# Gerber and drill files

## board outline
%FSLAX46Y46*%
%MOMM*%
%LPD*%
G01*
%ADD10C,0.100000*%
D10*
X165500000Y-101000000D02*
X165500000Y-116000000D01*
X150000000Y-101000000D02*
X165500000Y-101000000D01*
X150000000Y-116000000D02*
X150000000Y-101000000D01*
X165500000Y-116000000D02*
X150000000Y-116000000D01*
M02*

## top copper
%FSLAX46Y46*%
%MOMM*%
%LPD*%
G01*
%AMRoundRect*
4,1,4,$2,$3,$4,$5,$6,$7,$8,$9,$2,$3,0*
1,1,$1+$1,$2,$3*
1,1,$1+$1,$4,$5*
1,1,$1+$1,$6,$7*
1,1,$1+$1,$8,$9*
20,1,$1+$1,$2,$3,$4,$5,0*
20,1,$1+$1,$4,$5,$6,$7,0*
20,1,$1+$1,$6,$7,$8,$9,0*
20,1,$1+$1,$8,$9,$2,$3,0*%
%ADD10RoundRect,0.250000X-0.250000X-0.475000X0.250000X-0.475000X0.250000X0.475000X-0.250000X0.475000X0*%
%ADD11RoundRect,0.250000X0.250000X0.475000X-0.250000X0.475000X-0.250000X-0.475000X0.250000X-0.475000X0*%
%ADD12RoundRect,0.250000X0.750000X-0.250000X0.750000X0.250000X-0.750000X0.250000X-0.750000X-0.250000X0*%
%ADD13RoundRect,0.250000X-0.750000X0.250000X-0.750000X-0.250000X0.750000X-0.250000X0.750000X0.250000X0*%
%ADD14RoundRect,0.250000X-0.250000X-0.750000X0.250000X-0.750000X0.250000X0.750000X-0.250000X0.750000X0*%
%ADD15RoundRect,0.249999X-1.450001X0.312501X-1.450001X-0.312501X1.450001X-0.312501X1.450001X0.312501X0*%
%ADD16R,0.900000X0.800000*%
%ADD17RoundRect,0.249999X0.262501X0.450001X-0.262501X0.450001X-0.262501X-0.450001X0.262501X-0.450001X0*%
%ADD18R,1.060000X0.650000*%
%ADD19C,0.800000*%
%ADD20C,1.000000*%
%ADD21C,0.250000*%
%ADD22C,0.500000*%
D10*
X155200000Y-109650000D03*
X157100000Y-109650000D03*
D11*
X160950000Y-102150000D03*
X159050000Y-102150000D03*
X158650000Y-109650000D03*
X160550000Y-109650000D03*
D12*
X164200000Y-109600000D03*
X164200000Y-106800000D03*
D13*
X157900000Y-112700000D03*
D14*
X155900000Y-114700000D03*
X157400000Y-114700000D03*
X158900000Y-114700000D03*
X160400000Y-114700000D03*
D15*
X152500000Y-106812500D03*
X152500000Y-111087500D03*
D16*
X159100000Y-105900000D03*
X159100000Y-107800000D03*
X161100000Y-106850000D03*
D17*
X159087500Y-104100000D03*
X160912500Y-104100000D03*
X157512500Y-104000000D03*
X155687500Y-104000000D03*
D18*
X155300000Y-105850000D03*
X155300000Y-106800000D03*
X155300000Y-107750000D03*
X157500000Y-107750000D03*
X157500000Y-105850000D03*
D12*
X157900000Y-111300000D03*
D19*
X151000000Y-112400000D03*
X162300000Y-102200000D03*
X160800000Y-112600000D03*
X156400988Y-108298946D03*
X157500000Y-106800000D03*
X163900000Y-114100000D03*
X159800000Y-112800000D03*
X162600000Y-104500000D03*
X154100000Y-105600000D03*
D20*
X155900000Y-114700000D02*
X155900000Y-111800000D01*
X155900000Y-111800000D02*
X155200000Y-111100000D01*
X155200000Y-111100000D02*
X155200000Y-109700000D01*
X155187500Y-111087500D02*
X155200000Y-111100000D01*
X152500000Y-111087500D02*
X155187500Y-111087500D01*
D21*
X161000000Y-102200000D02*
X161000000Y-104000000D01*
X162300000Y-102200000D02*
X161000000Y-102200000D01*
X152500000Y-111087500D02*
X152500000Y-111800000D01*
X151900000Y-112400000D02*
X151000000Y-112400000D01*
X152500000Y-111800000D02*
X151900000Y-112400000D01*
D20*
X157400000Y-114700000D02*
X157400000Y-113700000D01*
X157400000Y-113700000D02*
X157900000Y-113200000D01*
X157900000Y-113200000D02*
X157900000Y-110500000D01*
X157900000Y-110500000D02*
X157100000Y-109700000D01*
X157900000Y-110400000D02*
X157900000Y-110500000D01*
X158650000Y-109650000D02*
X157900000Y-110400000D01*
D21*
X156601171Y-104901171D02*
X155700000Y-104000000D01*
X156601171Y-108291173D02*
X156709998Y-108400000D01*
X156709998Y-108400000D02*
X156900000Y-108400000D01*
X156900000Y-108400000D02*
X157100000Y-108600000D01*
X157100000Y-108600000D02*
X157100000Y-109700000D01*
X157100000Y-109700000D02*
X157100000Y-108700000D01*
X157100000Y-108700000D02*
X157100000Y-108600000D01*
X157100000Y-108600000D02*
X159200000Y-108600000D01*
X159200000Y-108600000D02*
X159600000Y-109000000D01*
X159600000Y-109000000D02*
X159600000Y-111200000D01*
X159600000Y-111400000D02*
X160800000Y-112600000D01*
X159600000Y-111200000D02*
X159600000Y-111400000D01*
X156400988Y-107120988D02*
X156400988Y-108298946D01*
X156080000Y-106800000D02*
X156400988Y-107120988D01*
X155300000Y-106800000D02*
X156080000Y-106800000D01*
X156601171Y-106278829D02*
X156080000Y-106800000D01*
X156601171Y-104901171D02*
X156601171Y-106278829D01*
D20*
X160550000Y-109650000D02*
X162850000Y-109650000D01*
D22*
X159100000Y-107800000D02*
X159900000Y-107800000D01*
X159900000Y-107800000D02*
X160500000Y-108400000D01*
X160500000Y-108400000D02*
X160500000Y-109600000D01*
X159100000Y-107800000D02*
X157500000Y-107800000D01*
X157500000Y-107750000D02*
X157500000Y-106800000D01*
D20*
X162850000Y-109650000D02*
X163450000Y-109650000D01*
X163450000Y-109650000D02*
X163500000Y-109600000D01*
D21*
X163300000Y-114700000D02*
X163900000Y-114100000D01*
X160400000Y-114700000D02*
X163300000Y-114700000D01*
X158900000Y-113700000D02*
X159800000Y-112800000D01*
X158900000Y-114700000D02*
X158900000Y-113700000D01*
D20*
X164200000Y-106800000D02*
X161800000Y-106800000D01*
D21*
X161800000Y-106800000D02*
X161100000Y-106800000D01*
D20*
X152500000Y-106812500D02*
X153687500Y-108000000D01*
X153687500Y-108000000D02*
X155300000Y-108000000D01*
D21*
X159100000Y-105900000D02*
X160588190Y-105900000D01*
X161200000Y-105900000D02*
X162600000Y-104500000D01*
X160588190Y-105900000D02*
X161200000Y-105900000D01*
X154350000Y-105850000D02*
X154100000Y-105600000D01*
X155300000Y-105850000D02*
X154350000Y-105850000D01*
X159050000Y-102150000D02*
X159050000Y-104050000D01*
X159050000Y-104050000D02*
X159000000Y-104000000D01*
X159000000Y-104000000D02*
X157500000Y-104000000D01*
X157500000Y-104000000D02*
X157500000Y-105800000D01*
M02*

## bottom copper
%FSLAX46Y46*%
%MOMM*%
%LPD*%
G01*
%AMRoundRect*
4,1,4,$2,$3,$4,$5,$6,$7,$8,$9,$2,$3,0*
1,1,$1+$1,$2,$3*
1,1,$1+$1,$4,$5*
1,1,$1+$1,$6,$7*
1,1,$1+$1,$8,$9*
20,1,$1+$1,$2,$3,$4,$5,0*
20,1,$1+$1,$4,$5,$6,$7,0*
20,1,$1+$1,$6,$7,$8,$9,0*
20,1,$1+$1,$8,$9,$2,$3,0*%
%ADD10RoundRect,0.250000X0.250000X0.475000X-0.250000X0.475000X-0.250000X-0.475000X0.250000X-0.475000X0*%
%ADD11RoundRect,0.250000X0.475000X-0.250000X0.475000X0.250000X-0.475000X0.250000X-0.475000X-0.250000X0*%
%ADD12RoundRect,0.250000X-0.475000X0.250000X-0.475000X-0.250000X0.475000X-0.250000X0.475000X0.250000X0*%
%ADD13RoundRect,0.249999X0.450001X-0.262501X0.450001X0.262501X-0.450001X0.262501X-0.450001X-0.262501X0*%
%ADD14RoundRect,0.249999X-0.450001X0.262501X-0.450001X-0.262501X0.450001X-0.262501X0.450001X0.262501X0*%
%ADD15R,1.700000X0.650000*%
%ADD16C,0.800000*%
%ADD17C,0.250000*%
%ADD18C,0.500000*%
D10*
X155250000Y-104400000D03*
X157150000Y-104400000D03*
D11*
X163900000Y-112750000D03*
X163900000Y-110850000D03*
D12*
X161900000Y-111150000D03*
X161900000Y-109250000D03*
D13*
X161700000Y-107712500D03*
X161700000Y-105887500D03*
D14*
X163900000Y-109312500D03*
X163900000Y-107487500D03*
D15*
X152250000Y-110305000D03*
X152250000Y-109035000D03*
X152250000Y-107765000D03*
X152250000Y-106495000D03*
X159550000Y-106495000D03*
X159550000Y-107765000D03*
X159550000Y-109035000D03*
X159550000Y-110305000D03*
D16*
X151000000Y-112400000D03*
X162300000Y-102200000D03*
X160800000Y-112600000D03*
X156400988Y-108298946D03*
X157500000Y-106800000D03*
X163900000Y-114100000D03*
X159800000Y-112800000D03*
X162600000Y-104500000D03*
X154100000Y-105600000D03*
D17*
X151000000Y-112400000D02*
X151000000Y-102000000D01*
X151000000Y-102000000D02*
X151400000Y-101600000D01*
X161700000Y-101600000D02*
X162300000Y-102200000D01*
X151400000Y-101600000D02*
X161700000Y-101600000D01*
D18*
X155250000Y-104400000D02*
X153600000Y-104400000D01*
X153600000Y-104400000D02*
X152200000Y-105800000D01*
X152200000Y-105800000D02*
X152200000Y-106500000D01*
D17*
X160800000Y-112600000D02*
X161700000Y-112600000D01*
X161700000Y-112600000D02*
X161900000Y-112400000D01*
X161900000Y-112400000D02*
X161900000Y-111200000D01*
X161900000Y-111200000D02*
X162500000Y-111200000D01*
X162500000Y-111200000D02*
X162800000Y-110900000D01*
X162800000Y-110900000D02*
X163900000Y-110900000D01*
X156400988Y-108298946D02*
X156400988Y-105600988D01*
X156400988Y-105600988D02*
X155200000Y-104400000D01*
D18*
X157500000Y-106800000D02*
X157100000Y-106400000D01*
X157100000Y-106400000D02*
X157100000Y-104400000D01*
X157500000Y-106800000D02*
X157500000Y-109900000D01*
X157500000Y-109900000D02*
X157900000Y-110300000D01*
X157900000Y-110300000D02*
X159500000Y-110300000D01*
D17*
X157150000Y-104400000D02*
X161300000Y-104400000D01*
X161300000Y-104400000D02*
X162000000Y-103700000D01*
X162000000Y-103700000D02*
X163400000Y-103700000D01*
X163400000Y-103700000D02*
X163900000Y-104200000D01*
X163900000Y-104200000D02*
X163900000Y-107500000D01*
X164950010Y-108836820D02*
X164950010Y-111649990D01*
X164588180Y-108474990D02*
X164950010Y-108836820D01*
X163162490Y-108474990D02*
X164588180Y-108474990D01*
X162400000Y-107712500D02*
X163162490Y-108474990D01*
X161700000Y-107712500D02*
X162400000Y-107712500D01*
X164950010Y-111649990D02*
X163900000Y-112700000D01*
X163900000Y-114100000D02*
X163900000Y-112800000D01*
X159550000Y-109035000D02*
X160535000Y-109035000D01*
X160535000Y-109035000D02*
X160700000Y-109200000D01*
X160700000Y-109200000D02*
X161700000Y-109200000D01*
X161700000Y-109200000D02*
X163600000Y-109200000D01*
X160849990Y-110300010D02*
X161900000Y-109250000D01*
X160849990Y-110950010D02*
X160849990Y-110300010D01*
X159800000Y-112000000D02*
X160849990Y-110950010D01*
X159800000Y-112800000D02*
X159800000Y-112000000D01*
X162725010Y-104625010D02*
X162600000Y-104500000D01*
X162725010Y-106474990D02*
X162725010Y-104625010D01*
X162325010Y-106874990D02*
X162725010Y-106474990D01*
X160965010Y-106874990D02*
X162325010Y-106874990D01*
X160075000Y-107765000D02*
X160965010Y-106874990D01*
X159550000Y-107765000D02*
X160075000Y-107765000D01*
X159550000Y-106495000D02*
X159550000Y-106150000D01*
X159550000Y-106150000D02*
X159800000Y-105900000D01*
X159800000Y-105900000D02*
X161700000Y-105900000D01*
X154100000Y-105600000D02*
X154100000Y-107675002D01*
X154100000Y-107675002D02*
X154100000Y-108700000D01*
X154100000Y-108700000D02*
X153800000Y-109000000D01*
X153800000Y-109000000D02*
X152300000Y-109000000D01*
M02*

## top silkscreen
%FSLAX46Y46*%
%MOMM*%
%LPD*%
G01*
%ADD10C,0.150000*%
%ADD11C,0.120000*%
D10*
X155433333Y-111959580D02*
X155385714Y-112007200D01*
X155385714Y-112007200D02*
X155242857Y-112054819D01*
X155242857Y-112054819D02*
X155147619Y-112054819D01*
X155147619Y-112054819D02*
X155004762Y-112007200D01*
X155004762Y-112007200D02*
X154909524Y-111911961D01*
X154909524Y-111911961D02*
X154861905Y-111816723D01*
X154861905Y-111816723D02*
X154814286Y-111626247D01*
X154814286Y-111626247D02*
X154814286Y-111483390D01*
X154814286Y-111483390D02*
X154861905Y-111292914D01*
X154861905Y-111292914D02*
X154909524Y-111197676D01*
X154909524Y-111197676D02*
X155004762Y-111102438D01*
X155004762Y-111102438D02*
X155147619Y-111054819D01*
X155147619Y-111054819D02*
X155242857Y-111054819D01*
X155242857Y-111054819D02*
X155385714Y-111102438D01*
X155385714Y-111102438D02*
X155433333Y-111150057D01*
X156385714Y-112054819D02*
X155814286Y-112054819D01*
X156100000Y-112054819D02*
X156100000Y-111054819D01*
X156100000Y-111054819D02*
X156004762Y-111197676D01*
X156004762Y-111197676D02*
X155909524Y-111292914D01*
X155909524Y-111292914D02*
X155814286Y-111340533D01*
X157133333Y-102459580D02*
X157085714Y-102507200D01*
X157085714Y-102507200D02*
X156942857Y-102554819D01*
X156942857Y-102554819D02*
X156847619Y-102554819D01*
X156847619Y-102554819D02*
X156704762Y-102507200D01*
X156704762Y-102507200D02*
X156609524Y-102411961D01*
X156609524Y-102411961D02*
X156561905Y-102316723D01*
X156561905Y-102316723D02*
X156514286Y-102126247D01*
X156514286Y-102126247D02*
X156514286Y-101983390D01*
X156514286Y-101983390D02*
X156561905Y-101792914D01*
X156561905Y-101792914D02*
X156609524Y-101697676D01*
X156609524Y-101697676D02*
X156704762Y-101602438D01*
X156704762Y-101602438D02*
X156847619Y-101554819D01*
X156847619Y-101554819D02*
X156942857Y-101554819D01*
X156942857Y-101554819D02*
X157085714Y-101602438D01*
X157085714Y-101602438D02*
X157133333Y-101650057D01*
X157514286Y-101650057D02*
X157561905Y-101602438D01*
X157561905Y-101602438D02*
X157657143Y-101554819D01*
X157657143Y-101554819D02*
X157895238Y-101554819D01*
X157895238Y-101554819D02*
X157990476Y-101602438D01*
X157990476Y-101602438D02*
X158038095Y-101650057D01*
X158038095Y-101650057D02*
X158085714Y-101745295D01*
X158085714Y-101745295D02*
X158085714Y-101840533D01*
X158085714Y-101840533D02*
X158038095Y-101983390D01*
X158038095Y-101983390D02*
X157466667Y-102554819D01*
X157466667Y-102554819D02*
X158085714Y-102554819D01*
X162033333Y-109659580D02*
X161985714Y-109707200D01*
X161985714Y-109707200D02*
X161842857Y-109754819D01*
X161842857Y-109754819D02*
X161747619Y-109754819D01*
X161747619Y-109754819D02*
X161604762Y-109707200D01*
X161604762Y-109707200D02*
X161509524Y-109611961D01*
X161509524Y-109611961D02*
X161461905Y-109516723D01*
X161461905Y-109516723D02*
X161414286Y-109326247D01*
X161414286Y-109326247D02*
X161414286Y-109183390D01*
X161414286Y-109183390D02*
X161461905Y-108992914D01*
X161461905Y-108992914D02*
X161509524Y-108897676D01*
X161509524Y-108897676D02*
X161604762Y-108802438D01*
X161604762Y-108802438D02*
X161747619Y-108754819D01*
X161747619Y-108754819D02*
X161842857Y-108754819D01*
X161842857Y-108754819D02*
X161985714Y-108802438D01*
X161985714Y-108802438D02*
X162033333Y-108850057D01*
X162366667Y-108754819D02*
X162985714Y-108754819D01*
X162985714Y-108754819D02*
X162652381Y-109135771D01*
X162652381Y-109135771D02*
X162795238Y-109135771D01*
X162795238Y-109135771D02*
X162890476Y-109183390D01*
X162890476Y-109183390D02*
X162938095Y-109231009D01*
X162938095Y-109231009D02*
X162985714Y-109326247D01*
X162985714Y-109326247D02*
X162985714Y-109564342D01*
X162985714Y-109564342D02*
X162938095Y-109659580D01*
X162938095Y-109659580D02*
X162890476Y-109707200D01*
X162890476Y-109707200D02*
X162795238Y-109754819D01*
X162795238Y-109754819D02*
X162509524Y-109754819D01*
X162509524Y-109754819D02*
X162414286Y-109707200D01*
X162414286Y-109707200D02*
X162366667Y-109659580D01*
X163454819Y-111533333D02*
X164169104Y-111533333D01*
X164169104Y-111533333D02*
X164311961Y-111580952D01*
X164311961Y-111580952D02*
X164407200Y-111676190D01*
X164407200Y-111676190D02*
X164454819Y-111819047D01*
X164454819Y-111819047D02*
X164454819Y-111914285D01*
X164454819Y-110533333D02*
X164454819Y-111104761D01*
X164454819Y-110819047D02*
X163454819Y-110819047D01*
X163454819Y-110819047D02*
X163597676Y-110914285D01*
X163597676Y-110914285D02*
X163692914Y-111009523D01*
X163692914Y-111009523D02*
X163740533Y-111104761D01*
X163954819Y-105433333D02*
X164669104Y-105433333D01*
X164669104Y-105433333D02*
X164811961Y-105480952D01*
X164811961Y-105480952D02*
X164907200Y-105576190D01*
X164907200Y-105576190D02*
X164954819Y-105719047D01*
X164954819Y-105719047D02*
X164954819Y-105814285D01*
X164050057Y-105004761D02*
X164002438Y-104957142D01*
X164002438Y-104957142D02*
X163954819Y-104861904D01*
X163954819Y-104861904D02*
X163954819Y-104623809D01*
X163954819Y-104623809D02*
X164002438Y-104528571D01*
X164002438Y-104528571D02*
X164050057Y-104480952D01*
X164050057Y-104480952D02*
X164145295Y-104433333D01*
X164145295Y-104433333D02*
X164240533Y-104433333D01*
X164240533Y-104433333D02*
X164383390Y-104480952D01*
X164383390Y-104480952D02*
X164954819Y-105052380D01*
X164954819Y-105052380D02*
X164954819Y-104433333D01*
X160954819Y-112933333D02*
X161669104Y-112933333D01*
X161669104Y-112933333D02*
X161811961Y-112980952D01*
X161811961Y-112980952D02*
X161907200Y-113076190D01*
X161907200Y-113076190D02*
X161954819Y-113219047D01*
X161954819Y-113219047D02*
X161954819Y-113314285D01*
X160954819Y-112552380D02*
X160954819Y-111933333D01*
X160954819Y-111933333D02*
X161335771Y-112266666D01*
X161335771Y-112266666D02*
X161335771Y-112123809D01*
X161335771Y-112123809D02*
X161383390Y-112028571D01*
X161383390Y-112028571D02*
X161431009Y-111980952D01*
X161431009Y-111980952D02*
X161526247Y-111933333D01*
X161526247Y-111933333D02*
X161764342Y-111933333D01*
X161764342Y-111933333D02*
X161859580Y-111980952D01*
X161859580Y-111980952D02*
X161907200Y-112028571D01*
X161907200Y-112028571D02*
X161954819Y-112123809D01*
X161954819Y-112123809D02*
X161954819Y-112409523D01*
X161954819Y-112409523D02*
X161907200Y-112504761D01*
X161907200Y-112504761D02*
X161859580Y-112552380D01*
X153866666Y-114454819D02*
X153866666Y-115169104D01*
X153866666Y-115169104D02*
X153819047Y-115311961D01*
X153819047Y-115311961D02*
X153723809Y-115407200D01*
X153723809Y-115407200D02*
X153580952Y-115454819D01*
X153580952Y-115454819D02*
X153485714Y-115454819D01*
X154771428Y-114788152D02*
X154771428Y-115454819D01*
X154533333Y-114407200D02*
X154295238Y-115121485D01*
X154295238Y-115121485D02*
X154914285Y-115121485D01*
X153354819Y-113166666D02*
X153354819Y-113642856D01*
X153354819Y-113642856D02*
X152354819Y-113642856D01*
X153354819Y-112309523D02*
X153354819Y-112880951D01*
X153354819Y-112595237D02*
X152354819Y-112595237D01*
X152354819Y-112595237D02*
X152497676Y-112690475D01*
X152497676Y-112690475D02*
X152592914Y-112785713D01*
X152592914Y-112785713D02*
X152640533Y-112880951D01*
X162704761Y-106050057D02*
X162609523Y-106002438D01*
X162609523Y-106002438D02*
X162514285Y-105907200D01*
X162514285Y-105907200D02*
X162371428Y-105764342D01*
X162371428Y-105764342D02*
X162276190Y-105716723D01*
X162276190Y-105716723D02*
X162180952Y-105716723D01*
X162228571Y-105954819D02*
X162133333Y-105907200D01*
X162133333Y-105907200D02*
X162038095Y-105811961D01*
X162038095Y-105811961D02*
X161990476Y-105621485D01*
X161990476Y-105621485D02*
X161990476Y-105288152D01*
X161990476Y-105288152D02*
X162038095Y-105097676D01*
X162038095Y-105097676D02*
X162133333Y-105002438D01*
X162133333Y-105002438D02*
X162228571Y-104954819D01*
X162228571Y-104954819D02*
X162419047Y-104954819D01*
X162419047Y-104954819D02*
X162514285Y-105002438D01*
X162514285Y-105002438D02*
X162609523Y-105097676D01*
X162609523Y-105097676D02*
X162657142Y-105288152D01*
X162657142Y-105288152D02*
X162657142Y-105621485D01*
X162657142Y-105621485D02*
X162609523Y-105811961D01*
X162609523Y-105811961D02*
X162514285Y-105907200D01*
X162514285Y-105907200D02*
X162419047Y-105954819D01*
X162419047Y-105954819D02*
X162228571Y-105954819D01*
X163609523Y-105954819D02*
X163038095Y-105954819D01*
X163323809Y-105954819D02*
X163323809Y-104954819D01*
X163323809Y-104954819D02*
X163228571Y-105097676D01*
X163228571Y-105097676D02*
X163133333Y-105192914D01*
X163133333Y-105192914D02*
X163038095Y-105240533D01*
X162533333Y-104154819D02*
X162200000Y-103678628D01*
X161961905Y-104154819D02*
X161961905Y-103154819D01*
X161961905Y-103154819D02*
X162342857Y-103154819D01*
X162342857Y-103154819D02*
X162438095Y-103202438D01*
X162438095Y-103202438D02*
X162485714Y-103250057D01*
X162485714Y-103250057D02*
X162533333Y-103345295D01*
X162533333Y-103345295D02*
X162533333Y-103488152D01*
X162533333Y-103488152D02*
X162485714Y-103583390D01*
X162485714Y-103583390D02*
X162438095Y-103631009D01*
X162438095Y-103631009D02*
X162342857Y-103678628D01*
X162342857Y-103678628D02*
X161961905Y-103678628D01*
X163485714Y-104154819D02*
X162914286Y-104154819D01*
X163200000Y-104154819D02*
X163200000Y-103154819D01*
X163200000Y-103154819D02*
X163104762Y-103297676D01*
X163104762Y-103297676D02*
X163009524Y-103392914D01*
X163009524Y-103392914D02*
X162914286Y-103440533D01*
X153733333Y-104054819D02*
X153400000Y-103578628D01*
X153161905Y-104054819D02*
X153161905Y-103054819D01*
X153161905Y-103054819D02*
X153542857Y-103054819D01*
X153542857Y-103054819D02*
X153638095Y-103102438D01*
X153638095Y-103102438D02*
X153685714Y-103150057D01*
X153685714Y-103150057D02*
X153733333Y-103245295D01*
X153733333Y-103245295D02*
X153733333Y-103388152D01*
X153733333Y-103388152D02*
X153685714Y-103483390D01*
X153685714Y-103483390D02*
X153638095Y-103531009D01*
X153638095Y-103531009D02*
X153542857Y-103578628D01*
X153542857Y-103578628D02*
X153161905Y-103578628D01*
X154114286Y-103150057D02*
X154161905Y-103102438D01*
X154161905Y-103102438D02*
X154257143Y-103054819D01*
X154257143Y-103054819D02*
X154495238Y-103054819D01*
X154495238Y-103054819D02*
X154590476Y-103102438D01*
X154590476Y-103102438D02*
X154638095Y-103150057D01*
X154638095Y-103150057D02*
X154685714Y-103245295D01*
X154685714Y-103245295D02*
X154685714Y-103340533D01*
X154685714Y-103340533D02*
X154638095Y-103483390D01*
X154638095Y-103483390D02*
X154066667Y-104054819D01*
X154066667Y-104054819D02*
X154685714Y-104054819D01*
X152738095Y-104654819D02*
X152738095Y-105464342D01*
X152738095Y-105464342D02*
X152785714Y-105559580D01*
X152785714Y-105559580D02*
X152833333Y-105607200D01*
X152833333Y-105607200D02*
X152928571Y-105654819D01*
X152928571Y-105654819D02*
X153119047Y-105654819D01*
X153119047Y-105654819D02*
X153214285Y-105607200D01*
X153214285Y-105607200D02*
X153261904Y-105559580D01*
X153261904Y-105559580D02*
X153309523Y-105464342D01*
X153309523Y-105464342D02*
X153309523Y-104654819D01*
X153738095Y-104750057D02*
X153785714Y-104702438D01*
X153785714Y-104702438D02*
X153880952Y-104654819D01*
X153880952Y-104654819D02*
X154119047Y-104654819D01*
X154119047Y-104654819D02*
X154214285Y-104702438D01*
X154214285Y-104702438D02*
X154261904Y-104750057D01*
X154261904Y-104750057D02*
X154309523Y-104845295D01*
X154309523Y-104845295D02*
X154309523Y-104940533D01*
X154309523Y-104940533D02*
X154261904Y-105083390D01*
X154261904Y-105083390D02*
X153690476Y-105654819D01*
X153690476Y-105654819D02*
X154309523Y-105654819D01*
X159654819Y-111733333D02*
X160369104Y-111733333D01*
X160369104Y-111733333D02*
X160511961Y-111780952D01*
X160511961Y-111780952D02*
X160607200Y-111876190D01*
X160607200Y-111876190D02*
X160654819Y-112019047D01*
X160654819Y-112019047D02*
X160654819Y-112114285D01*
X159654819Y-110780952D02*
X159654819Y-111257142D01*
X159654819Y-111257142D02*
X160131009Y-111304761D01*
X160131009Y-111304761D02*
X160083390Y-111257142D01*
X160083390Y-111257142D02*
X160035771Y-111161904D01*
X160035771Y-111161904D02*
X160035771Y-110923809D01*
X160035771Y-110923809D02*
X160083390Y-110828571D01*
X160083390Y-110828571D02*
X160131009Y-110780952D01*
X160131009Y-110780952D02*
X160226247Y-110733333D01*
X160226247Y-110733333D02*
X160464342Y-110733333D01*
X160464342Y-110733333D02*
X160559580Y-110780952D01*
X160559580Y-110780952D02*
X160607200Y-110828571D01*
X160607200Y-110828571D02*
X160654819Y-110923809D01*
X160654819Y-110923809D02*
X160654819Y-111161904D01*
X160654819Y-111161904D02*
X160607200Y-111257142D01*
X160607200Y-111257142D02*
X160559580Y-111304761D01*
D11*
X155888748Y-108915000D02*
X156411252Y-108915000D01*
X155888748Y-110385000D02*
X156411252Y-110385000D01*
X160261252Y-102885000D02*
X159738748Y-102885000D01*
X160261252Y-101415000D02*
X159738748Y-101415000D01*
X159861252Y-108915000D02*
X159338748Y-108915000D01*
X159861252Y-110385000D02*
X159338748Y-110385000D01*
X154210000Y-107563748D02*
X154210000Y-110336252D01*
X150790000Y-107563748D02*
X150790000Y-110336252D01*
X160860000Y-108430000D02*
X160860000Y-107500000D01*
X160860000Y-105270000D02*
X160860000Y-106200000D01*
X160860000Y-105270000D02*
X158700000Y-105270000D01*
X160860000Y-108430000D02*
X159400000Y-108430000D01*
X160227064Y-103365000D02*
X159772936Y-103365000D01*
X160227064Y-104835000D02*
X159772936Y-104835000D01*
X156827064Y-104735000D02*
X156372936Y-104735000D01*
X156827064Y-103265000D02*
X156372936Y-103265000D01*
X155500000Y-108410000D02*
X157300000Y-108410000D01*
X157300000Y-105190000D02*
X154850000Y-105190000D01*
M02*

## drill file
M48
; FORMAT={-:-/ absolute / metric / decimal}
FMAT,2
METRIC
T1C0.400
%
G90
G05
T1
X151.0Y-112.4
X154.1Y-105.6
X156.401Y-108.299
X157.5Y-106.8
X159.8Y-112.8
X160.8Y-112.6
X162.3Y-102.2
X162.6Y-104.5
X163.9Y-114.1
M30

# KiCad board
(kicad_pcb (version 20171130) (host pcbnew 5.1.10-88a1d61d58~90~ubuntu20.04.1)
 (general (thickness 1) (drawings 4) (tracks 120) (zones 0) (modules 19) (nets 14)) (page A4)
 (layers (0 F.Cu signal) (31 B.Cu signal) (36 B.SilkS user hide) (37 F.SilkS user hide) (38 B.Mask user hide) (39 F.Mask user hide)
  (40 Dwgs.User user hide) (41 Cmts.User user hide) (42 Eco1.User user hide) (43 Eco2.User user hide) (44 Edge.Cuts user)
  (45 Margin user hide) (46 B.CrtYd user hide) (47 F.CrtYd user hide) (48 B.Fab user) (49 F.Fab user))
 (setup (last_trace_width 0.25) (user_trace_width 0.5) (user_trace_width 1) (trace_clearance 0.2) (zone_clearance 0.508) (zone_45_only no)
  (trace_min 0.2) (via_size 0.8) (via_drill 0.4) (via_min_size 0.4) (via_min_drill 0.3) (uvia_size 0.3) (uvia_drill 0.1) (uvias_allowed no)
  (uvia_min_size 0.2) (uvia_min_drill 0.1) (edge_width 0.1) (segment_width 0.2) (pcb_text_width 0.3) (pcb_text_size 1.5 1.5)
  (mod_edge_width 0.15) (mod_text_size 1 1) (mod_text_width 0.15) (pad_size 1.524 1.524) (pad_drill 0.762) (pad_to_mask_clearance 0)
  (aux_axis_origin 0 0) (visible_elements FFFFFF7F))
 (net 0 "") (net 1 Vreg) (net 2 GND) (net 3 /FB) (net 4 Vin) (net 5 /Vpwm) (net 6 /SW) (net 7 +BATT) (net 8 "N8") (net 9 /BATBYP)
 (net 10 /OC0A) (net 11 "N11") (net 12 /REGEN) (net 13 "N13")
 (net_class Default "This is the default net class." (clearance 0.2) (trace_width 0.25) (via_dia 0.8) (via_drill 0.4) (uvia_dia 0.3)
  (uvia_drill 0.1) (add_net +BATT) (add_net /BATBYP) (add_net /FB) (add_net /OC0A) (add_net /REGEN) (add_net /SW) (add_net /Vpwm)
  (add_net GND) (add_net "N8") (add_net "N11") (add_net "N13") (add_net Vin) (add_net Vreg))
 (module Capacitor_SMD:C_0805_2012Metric (layer F.Cu) (at 156.15 109.65)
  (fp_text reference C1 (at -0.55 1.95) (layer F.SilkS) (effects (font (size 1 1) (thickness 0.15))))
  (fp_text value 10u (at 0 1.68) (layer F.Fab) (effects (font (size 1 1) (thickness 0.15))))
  (fp_line (start -0.261252 -0.735) (end 0.261252 -0.735) (layer F.SilkS) (width 0.12))
  (fp_line (start -0.261252 0.735) (end 0.261252 0.735) (layer F.SilkS) (width 0.12))
  (pad 1 smd roundrect (at -0.95 0) (size 1 1.45) (layers F.Cu F.Paste F.Mask) (roundrect_rratio 0.25) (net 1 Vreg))
  (pad 2 smd roundrect (at 0.95 0) (size 1 1.45) (layers F.Cu F.Paste F.Mask) (roundrect_rratio 0.25) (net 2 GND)))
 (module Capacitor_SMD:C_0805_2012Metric (layer F.Cu) (at 160 102.15 180)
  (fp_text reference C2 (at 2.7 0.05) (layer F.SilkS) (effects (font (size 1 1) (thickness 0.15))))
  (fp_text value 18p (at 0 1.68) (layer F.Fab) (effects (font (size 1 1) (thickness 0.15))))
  (fp_line (start -0.261252 -0.735) (end 0.261252 -0.735) (layer F.SilkS) (width 0.12))
  (fp_line (start -0.261252 0.735) (end 0.261252 0.735) (layer F.SilkS) (width 0.12))
  (pad 1 smd roundrect (at -0.95 0 180) (size 1 1.45) (layers F.Cu F.Paste F.Mask) (roundrect_rratio 0.25) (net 1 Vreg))
  (pad 2 smd roundrect (at 0.95 0 180) (size 1 1.45) (layers F.Cu F.Paste F.Mask) (roundrect_rratio 0.25) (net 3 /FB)))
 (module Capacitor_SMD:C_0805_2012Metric (layer F.Cu) (at 159.6 109.65 180)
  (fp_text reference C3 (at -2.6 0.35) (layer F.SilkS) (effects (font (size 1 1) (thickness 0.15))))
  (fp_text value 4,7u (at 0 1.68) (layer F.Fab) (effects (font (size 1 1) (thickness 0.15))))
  (fp_line (start -0.261252 0.735) (end 0.261252 0.735) (layer F.SilkS) (width 0.12))
  (fp_line (start -0.261252 -0.735) (end 0.261252 -0.735) (layer F.SilkS) (width 0.12))
  (pad 2 smd roundrect (at 0.95 0 180) (size 1 1.45) (layers F.Cu F.Paste F.Mask) (roundrect_rratio 0.25) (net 2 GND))
  (pad 1 smd roundrect (at -0.95 0 180) (size 1 1.45) (layers F.Cu F.Paste F.Mask) (roundrect_rratio 0.25) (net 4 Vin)))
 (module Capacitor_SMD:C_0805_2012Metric (layer B.Cu) (at 156.2 104.4 180)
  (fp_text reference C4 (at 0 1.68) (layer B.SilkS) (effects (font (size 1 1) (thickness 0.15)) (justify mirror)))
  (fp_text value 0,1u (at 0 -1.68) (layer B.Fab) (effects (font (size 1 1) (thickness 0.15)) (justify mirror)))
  (pad 2 smd roundrect (at 0.95 0 180) (size 1 1.45) (layers B.Cu B.Paste B.Mask) (roundrect_rratio 0.25) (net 2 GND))
  (pad 1 smd roundrect (at -0.95 0 180) (size 1 1.45) (layers B.Cu B.Paste B.Mask) (roundrect_rratio 0.25) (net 4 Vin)))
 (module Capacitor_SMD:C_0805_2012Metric (layer B.Cu) (at 163.9 111.8 90)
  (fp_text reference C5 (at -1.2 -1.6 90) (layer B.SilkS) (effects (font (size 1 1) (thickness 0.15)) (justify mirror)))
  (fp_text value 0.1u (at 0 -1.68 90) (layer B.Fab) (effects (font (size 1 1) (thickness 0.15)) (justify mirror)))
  (pad 1 smd roundrect (at -0.95 0 90) (size 1 1.45) (layers B.Cu B.Paste B.Mask) (roundrect_rratio 0.25) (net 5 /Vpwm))
  (pad 2 smd roundrect (at 0.95 0 90) (size 1 1.45) (layers B.Cu B.Paste B.Mask) (roundrect_rratio 0.25) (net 2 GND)))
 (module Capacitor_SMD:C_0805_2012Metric (layer B.Cu) (at 161.9 110.2 270)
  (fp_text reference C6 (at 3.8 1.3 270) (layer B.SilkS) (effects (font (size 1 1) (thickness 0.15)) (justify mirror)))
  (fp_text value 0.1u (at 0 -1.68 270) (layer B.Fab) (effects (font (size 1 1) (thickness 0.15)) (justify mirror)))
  (pad 2 smd roundrect (at 0.95 0 270) (size 1 1.45) (layers B.Cu B.Paste B.Mask) (roundrect_rratio 0.25) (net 2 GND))
  (pad 1 smd roundrect (at -0.95 0 270) (size 1 1.45) (layers B.Cu B.Paste B.Mask) (roundrect_rratio 0.25) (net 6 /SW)))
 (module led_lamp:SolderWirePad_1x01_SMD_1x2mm (layer F.Cu) (at 164.2 109.6 90)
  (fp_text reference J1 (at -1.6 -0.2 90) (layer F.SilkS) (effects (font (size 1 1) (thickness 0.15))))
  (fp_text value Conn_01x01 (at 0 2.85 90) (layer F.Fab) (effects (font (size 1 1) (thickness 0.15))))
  (pad 1 smd roundrect (at 0 0 90) (size 1 2) (layers F.Cu F.Paste F.Mask) (roundrect_rratio 0.25) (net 4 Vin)))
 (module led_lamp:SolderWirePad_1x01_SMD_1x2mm (layer F.Cu) (at 164.2 106.8 90)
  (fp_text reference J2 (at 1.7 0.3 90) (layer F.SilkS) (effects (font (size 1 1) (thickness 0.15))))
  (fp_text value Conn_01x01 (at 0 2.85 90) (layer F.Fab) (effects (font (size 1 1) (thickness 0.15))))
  (pad 1 smd roundrect (at 0 0 90) (size 1 2) (layers F.Cu F.Paste F.Mask) (roundrect_rratio 0.25) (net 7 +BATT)))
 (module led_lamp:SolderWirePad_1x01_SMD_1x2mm (layer F.Cu) (at 157.9 112.7 270)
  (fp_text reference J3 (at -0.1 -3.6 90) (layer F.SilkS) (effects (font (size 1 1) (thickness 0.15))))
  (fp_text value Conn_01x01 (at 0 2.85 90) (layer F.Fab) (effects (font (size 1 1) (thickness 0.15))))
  (pad 1 smd roundrect (at 0 0 270) (size 1 2) (layers F.Cu F.Paste F.Mask) (roundrect_rratio 0.25) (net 2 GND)))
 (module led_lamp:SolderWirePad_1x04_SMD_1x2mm (layer F.Cu) (at 155.9 114.7)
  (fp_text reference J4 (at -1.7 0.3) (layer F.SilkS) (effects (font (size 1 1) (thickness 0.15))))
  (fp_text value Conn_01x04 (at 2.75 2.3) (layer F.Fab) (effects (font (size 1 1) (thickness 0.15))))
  (pad 1 smd roundrect (at 0 0) (size 1 2) (layers F.Cu F.Paste F.Mask) (roundrect_rratio 0.25) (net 1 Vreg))
  (pad 2 smd roundrect (at 1.5 0) (size 1 2) (layers F.Cu F.Paste F.Mask) (roundrect_rratio 0.25) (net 2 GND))
  (pad 3 smd roundrect (at 3 0) (size 1 2) (layers F.Cu F.Paste F.Mask) (roundrect_rratio 0.25) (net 6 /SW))
  (pad 4 smd roundrect (at 4.5 0) (size 1 2) (layers F.Cu F.Paste F.Mask) (roundrect_rratio 0.25) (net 5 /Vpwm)))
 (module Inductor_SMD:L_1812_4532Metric (layer F.Cu) (at 152.5 108.95 270)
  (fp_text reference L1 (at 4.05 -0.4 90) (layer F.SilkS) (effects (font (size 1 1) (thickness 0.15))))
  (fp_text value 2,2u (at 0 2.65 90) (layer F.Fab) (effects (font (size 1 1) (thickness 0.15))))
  (fp_line (start -1.386252 -1.71) (end 1.386252 -1.71) (layer F.SilkS) (width 0.12))
  (fp_line (start -1.386252 1.71) (end 1.386252 1.71) (layer F.SilkS) (width 0.12))
  (pad 1 smd roundrect (at -2.1375 0 270) (size 1.125 3.4) (layers F.Cu F.Paste F.Mask) (roundrect_rratio 0.2222213333333333) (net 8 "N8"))
  (pad 2 smd roundrect (at 2.1375 0 270) (size 1.125 3.4) (layers F.Cu F.Paste F.Mask) (roundrect_rratio 0.2222213333333333) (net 1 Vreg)))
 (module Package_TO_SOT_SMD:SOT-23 (layer F.Cu) (at 160.1 106.85)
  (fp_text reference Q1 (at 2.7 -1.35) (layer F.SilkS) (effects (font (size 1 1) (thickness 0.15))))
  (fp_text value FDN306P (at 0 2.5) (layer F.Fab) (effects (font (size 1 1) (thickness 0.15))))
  (fp_line (start 0.76 1.58) (end 0.76 0.65) (layer F.SilkS) (width 0.12))
  (fp_line (start 0.76 -1.58) (end 0.76 -0.65) (layer F.SilkS) (width 0.12))
  (fp_line (start 0.76 -1.58) (end -1.4 -1.58) (layer F.SilkS) (width 0.12))
  (fp_line (start 0.76 1.58) (end -0.7 1.58) (layer F.SilkS) (width 0.12))
  (pad 1 smd rect (at -1 -0.95) (size 0.9 0.8) (layers F.Cu F.Paste F.Mask) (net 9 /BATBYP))
  (pad 2 smd rect (at -1 0.95) (size 0.9 0.8) (layers F.Cu F.Paste F.Mask) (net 4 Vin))
  (pad 3 smd rect (at 1 0) (size 0.9 0.8) (layers F.Cu F.Paste F.Mask) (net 7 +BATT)))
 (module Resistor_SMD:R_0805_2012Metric (layer F.Cu) (at 160 104.1 180)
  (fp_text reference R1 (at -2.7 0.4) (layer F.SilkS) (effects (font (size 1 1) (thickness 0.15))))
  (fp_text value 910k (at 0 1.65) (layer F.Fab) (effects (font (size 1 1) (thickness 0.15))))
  (fp_line (start -0.227064 0.735) (end 0.227064 0.735) (layer F.SilkS) (width 0.12))
  (fp_line (start -0.227064 -0.735) (end 0.227064 -0.735) (layer F.SilkS) (width 0.12))
  (pad 2 smd roundrect (at 0.9125 0 180) (size 1.025 1.4) (layers F.Cu F.Paste F.Mask) (roundrect_rratio 0.2439014634146341) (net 3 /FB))
  (pad 1 smd roundrect (at -0.9125 0 180) (size 1.025 1.4) (layers F.Cu F.Paste F.Mask) (roundrect_rratio 0.2439014634146341) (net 1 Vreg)))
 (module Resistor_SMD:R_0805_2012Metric (layer F.Cu) (at 156.6 104 180)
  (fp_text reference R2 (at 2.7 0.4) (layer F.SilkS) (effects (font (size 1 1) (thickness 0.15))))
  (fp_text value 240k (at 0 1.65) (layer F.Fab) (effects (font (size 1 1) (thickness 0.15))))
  (fp_line (start -0.227064 -0.735) (end 0.227064 -0.735) (layer F.SilkS) (width 0.12))
  (fp_line (start -0.227064 0.735) (end 0.227064 0.735) (layer F.SilkS) (width 0.12))
  (pad 1 smd roundrect (at -0.9125 0 180) (size 1.025 1.4) (layers F.Cu F.Paste F.Mask) (roundrect_rratio 0.2439014634146341) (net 3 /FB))
  (pad 2 smd roundrect (at 0.9125 0 180) (size 1.025 1.4) (layers F.Cu F.Paste F.Mask) (roundrect_rratio 0.2439014634146341) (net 2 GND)))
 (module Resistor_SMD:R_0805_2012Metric (layer B.Cu) (at 161.7 106.8 90)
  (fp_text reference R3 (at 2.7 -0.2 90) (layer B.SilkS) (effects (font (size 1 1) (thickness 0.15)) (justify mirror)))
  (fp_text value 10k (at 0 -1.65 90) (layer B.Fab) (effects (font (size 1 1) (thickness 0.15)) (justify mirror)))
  (pad 1 smd roundrect (at -0.9125 0 90) (size 1.025 1.4) (layers B.Cu B.Paste B.Mask) (roundrect_rratio 0.2439014634146341) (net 5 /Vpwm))
  (pad 2 smd roundrect (at 0.9125 0 90) (size 1.025 1.4) (layers B.Cu B.Paste B.Mask) (roundrect_rratio 0.2439014634146341) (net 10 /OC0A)))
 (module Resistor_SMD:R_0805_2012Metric (layer B.Cu) (at 163.9 108.4 270)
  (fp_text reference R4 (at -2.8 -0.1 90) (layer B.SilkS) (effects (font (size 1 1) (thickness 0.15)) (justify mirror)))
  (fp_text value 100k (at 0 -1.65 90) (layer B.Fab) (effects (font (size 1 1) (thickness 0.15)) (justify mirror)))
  (pad 2 smd roundrect (at 0.9125 0 270) (size 1.025 1.4) (layers B.Cu B.Paste B.Mask) (roundrect_rratio 0.2439014634146341) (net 6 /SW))
  (pad 1 smd roundrect (at -0.9125 0 270) (size 1.025 1.4) (layers B.Cu B.Paste B.Mask) (roundrect_rratio 0.2439014634146341) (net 4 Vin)))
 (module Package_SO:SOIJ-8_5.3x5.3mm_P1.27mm (layer B.Cu) (at 155.9 108.4)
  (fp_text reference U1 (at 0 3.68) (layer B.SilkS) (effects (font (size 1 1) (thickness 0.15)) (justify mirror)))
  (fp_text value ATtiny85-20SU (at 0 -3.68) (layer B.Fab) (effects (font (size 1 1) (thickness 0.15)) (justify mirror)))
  (pad 1 smd rect (at -3.65 1.905) (size 1.7 0.65) (layers B.Cu B.Paste B.Mask) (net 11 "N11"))
  (pad 2 smd rect (at -3.65 0.635) (size 1.7 0.65) (layers B.Cu B.Paste B.Mask) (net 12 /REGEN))
  (pad 3 smd rect (at -3.65 -0.635) (size 1.7 0.65) (layers B.Cu B.Paste B.Mask) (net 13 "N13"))
  (pad 4 smd rect (at -3.65 -1.905) (size 1.7 0.65) (layers B.Cu B.Paste B.Mask) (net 2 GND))
  (pad 5 smd rect (at 3.65 -1.905) (size 1.7 0.65) (layers B.Cu B.Paste B.Mask) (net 10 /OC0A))
  (pad 6 smd rect (at 3.65 -0.635) (size 1.7 0.65) (layers B.Cu B.Paste B.Mask) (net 9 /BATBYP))
  (pad 7 smd rect (at 3.65 0.635) (size 1.7 0.65) (layers B.Cu B.Paste B.Mask) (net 6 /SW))
  (pad 8 smd rect (at 3.65 1.905) (size 1.7 0.65) (layers B.Cu B.Paste B.Mask) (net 4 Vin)))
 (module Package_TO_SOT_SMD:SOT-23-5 (layer F.Cu) (at 156.4 106.8)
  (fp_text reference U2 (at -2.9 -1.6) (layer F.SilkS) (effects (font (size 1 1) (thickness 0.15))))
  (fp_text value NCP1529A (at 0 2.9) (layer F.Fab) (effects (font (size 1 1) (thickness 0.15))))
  (fp_line (start -0.9 1.61) (end 0.9 1.61) (layer F.SilkS) (width 0.12))
  (fp_line (start 0.9 -1.61) (end -1.55 -1.61) (layer F.SilkS) (width 0.12))
  (pad 1 smd rect (at -1.1 -0.95) (size 1.06 0.65) (layers F.Cu F.Paste F.Mask) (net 12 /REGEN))
  (pad 2 smd rect (at -1.1 0) (size 1.06 0.65) (layers F.Cu F.Paste F.Mask) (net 2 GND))
  (pad 3 smd rect (at -1.1 0.95) (size 1.06 0.65) (layers F.Cu F.Paste F.Mask) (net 8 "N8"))
  (pad 4 smd rect (at 1.1 0.95) (size 1.06 0.65) (layers F.Cu F.Paste F.Mask) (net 4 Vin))
  (pad 5 smd rect (at 1.1 -0.95) (size 1.06 0.65) (layers F.Cu F.Paste F.Mask) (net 3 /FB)))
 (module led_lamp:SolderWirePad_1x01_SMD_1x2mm (layer F.Cu) (at 157.9 111.3 90)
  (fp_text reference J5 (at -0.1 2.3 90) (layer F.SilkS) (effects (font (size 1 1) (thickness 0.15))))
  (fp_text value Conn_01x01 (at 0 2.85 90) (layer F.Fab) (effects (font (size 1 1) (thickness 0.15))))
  (pad 1 smd roundrect (at 0 0 90) (size 1 2) (layers F.Cu F.Paste F.Mask) (roundrect_rratio 0.25) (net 2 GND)))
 (gr_line (start 165.5 101) (end 165.5 116) (layer Edge.Cuts) (width 0.1))
 (gr_line (start 150 101) (end 165.5 101) (layer Edge.Cuts) (width 0.1))
 (gr_line (start 150 116) (end 150 101) (layer Edge.Cuts) (width 0.1))
 (gr_line (start 165.5 116) (end 150 116) (layer Edge.Cuts) (width 0.1))
 (segment (start 155.9 114.7) (end 155.9 111.8) (width 1) (layer F.Cu) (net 1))
 (segment (start 155.9 111.8) (end 155.2 111.1) (width 1) (layer F.Cu) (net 1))
 (segment (start 155.2 111.1) (end 155.2 109.7) (width 1) (layer F.Cu) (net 1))
 (segment (start 155.1875 111.0875) (end 155.2 111.1) (width 1) (layer F.Cu) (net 1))
 (segment (start 152.5 111.0875) (end 155.1875 111.0875) (width 1) (layer F.Cu) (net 1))
 (segment (start 161 102.2) (end 161 104) (width 0.25) (layer F.Cu) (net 1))
 (via (at 151 112.4) (size 0.8) (drill 0.4) (layers F.Cu B.Cu) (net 1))
 (segment (start 162.3 102.2) (end 161 102.2) (width 0.25) (layer F.Cu) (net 1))
 (via (at 162.3 102.2) (size 0.8) (drill 0.4) (layers F.Cu B.Cu) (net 1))
 (segment (start 152.5 111.0875) (end 152.5 111.8) (width 0.25) (layer F.Cu) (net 1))
 (segment (start 151.9 112.4) (end 151 112.4) (width 0.25) (layer F.Cu) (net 1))
 (segment (start 152.5 111.8) (end 151.9 112.4) (width 0.25) (layer F.Cu) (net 1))
 (segment (start 151 112.4) (end 151 102) (width 0.25) (layer B.Cu) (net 1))
 (segment (start 151 102) (end 151.4 101.6) (width 0.25) (layer B.Cu) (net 1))
 (segment (start 161.7 101.6) (end 162.3 102.2) (width 0.25) (layer B.Cu) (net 1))
 (segment (start 151.4 101.6) (end 161.7 101.6) (width 0.25) (layer B.Cu) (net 1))
 (segment (start 157.4 114.7) (end 157.4 113.7) (width 1) (layer F.Cu) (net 2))
 (segment (start 157.4 113.7) (end 157.9 113.2) (width 1) (layer F.Cu) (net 2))
 (segment (start 157.9 113.2) (end 157.9 110.5) (width 1) (layer F.Cu) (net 2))
 (segment (start 157.9 110.5) (end 157.1 109.7) (width 1) (layer F.Cu) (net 2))
 (segment (start 157.9 110.4) (end 157.9 110.5) (width 1) (layer F.Cu) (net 2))
 (segment (start 158.65 109.65) (end 157.9 110.4) (width 1) (layer F.Cu) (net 2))
 (segment (start 156.601171 104.901171) (end 155.7 104) (width 0.25) (layer F.Cu) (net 2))
 (segment (start 155.25 104.4) (end 153.6 104.4) (width 0.5) (layer B.Cu) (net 2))
 (segment (start 153.6 104.4) (end 152.2 105.8) (width 0.5) (layer B.Cu) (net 2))
 (segment (start 152.2 105.8) (end 152.2 106.5) (width 0.5) (layer B.Cu) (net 2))
 (segment (start 156.601171 108.291173) (end 156.709998 108.4) (width 0.25) (layer F.Cu) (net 2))
 (segment (start 156.709998 108.4) (end 156.9 108.4) (width 0.25) (layer F.Cu) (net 2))
 (segment (start 156.9 108.4) (end 157.1 108.6) (width 0.25) (layer F.Cu) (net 2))
 (segment (start 157.1 108.6) (end 157.1 109.7) (width 0.25) (layer F.Cu) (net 2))
 (segment (start 157.1 109.7) (end 157.1 108.7) (width 0.25) (layer F.Cu) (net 2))
 (segment (start 157.1 108.7) (end 157.1 108.6) (width 0.25) (layer F.Cu) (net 2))
 (segment (start 157.1 108.6) (end 159.2 108.6) (width 0.25) (layer F.Cu) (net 2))
 (segment (start 159.2 108.6) (end 159.6 109) (width 0.25) (layer F.Cu) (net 2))
 (segment (start 159.6 109) (end 159.6 111.2) (width 0.25) (layer F.Cu) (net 2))
 (via (at 160.8 112.6) (size 0.8) (drill 0.4) (layers F.Cu B.Cu) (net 2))
 (segment (start 159.6 111.4) (end 160.8 112.6) (width 0.25) (layer F.Cu) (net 2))
 (segment (start 159.6 111.2) (end 159.6 111.4) (width 0.25) (layer F.Cu) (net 2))
 (segment (start 160.8 112.6) (end 161.7 112.6) (width 0.25) (layer B.Cu) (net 2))
 (segment (start 161.7 112.6) (end 161.9 112.4) (width 0.25) (layer B.Cu) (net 2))
 (segment (start 161.9 112.4) (end 161.9 111.2) (width 0.25) (layer B.Cu) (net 2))
 (segment (start 161.9 111.2) (end 162.5 111.2) (width 0.25) (layer B.Cu) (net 2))
 (segment (start 162.5 111.2) (end 162.8 110.9) (width 0.25) (layer B.Cu) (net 2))
 (segment (start 162.8 110.9) (end 163.9 110.9) (width 0.25) (layer B.Cu) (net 2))
 (via (at 156.400988 108.298946) (size 0.8) (drill 0.4) (layers F.Cu B.Cu) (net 2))
 (segment (start 156.400988 107.120988) (end 156.400988 108.298946) (width 0.25) (layer F.Cu) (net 2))
 (segment (start 156.08 106.8) (end 156.400988 107.120988) (width 0.25) (layer F.Cu) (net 2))
 (segment (start 155.3 106.8) (end 156.08 106.8) (width 0.25) (layer F.Cu) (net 2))
 (segment (start 156.400988 108.298946) (end 156.400988 105.600988) (width 0.25) (layer B.Cu) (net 2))
 (segment (start 156.400988 105.600988) (end 155.2 104.4) (width 0.25) (layer B.Cu) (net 2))
 (segment (start 156.601171 106.278829) (end 156.08 106.8) (width 0.25) (layer F.Cu) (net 2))
 (segment (start 156.601171 104.901171) (end 156.601171 106.278829) (width 0.25) (layer F.Cu) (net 2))
 (segment (start 160.55 109.65) (end 162.85 109.65) (width 1) (layer F.Cu) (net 4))
 (segment (start 159.1 107.8) (end 159.9 107.8) (width 0.5) (layer F.Cu) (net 4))
 (segment (start 159.9 107.8) (end 160.5 108.4) (width 0.5) (layer F.Cu) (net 4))
 (segment (start 160.5 108.4) (end 160.5 109.6) (width 0.5) (layer F.Cu) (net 4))
 (segment (start 159.1 107.8) (end 157.5 107.8) (width 0.5) (layer F.Cu) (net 4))
 (via (at 157.5 106.8) (size 0.8) (drill 0.4) (layers F.Cu B.Cu) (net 4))
 (segment (start 157.5 107.75) (end 157.5 106.8) (width 0.5) (layer F.Cu) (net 4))
 (segment (start 157.5 106.8) (end 157.1 106.4) (width 0.5) (layer B.Cu) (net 4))
 (segment (start 157.1 106.4) (end 157.1 104.4) (width 0.5) (layer B.Cu) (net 4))
 (segment (start 157.5 106.8) (end 157.5 109.9) (width 0.5) (layer B.Cu) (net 4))
 (segment (start 157.5 109.9) (end 157.9 110.3) (width 0.5) (layer B.Cu) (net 4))
 (segment (start 157.9 110.3) (end 159.5 110.3) (width 0.5) (layer B.Cu) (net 4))
 (segment (start 162.85 109.65) (end 163.45 109.65) (width 1) (layer F.Cu) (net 4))
 (segment (start 163.45 109.65) (end 163.5 109.6) (width 1) (layer F.Cu) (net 4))
 (segment (start 157.15 104.4) (end 161.3 104.4) (width 0.25) (layer B.Cu) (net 4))
 (segment (start 161.3 104.4) (end 162 103.7) (width 0.25) (layer B.Cu) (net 4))
 (segment (start 162 103.7) (end 163.4 103.7) (width 0.25) (layer B.Cu) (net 4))
 (segment (start 163.4 103.7) (end 163.9 104.2) (width 0.25) (layer B.Cu) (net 4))
 (segment (start 163.9 104.2) (end 163.9 107.5) (width 0.25) (layer B.Cu) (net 4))
 (segment (start 164.95001 108.83682) (end 164.95001 111.64999) (width 0.25) (layer B.Cu) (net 5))
 (segment (start 164.58818 108.47499) (end 164.95001 108.83682) (width 0.25) (layer B.Cu) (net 5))
 (segment (start 163.16249 108.47499) (end 164.58818 108.47499) (width 0.25) (layer B.Cu) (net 5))
 (segment (start 162.4 107.7125) (end 163.16249 108.47499) (width 0.25) (layer B.Cu) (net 5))
 (segment (start 161.7 107.7125) (end 162.4 107.7125) (width 0.25) (layer B.Cu) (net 5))
 (segment (start 164.95001 111.64999) (end 163.9 112.7) (width 0.25) (layer B.Cu) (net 5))
 (via (at 163.9 114.1) (size 0.8) (drill 0.4) (layers F.Cu B.Cu) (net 5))
 (segment (start 163.3 114.7) (end 163.9 114.1) (width 0.25) (layer F.Cu) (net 5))
 (segment (start 160.4 114.7) (end 163.3 114.7) (width 0.25) (layer F.Cu) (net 5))
 (segment (start 163.9 114.1) (end 163.9 112.8) (width 0.25) (layer B.Cu) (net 5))
 (segment (start 159.55 109.035) (end 160.535 109.035) (width 0.25) (layer B.Cu) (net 6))
 (segment (start 160.535 109.035) (end 160.7 109.2) (width 0.25) (layer B.Cu) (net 6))
 (segment (start 160.7 109.2) (end 161.7 109.2) (width 0.25) (layer B.Cu) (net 6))
 (segment (start 161.7 109.2) (end 163.6 109.2) (width 0.25) (layer B.Cu) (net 6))
 (via (at 159.8 112.8) (size 0.8) (drill 0.4) (layers F.Cu B.Cu) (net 6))
 (segment (start 158.9 113.7) (end 159.8 112.8) (width 0.25) (layer F.Cu) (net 6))
 (segment (start 158.9 114.7) (end 158.9 113.7) (width 0.25) (layer F.Cu) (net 6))
 (segment (start 160.84999 110.30001) (end 161.9 109.25) (width 0.25) (layer B.Cu) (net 6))
 (segment (start 160.84999 110.95001) (end 160.84999 110.30001) (width 0.25) (layer B.Cu) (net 6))
 (segment (start 159.8 112) (end 160.84999 110.95001) (width 0.25) (layer B.Cu) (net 6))
 (segment (start 159.8 112.8) (end 159.8 112) (width 0.25) (layer B.Cu) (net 6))
 (segment (start 164.2 106.8) (end 161.8 106.8) (width 1) (layer F.Cu) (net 7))
 (segment (start 161.8 106.8) (end 161.1 106.8) (width 0.25) (layer F.Cu) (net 7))
 (segment (start 152.5 106.8125) (end 153.6875 108) (width 1) (layer F.Cu) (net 8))
 (segment (start 153.6875 108) (end 155.3 108) (width 1) (layer F.Cu) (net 8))
 (segment (start 159.1 105.9) (end 160.58819 105.9) (width 0.25) (layer F.Cu) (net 9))
 (via (at 162.6 104.5) (size 0.8) (drill 0.4) (layers F.Cu B.Cu) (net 9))
 (segment (start 161.2 105.9) (end 162.6 104.5) (width 0.25) (layer F.Cu) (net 9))
 (segment (start 160.58819 105.9) (end 161.2 105.9) (width 0.25) (layer F.Cu) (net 9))
 (segment (start 162.72501 104.62501) (end 162.6 104.5) (width 0.25) (layer B.Cu) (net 9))
 (segment (start 162.72501 106.47499) (end 162.72501 104.62501) (width 0.25) (layer B.Cu) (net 9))
 (segment (start 162.32501 106.87499) (end 162.72501 106.47499) (width 0.25) (layer B.Cu) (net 9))
 (segment (start 160.96501 106.87499) (end 162.32501 106.87499) (width 0.25) (layer B.Cu) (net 9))
 (segment (start 160.075 107.765) (end 160.96501 106.87499) (width 0.25) (layer B.Cu) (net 9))
 (segment (start 159.55 107.765) (end 160.075 107.765) (width 0.25) (layer B.Cu) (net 9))
 (segment (start 159.55 106.495) (end 159.55 106.15) (width 0.25) (layer B.Cu) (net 10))
 (segment (start 159.55 106.15) (end 159.8 105.9) (width 0.25) (layer B.Cu) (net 10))
 (segment (start 159.8 105.9) (end 161.7 105.9) (width 0.25) (layer B.Cu) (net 10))
 (via (at 154.1 105.6) (size 0.8) (drill 0.4) (layers F.Cu B.Cu) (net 12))
 (segment (start 154.35 105.85) (end 154.1 105.6) (width 0.25) (layer F.Cu) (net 12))
 (segment (start 155.3 105.85) (end 154.35 105.85) (width 0.25) (layer F.Cu) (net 12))
 (segment (start 154.1 105.6) (end 154.1 107.675002) (width 0.25) (layer B.Cu) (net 12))
 (segment (start 154.1 107.675002) (end 154.1 108.7) (width 0.25) (layer B.Cu) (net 12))
 (segment (start 154.1 108.7) (end 153.8 109) (width 0.25) (layer B.Cu) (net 12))
 (segment (start 153.8 109) (end 152.3 109) (width 0.25) (layer B.Cu) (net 12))
 (segment (start 159.05 102.15) (end 159.05 104.05) (width 0.25) (layer F.Cu) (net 3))
 (segment (start 159.05 104.05) (end 159 104) (width 0.25) (layer F.Cu) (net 3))
 (segment (start 159 104) (end 157.5 104) (width 0.25) (layer F.Cu) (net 3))
 (segment (start 157.5 104) (end 157.5 105.8) (width 0.25) (layer F.Cu) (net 3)))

